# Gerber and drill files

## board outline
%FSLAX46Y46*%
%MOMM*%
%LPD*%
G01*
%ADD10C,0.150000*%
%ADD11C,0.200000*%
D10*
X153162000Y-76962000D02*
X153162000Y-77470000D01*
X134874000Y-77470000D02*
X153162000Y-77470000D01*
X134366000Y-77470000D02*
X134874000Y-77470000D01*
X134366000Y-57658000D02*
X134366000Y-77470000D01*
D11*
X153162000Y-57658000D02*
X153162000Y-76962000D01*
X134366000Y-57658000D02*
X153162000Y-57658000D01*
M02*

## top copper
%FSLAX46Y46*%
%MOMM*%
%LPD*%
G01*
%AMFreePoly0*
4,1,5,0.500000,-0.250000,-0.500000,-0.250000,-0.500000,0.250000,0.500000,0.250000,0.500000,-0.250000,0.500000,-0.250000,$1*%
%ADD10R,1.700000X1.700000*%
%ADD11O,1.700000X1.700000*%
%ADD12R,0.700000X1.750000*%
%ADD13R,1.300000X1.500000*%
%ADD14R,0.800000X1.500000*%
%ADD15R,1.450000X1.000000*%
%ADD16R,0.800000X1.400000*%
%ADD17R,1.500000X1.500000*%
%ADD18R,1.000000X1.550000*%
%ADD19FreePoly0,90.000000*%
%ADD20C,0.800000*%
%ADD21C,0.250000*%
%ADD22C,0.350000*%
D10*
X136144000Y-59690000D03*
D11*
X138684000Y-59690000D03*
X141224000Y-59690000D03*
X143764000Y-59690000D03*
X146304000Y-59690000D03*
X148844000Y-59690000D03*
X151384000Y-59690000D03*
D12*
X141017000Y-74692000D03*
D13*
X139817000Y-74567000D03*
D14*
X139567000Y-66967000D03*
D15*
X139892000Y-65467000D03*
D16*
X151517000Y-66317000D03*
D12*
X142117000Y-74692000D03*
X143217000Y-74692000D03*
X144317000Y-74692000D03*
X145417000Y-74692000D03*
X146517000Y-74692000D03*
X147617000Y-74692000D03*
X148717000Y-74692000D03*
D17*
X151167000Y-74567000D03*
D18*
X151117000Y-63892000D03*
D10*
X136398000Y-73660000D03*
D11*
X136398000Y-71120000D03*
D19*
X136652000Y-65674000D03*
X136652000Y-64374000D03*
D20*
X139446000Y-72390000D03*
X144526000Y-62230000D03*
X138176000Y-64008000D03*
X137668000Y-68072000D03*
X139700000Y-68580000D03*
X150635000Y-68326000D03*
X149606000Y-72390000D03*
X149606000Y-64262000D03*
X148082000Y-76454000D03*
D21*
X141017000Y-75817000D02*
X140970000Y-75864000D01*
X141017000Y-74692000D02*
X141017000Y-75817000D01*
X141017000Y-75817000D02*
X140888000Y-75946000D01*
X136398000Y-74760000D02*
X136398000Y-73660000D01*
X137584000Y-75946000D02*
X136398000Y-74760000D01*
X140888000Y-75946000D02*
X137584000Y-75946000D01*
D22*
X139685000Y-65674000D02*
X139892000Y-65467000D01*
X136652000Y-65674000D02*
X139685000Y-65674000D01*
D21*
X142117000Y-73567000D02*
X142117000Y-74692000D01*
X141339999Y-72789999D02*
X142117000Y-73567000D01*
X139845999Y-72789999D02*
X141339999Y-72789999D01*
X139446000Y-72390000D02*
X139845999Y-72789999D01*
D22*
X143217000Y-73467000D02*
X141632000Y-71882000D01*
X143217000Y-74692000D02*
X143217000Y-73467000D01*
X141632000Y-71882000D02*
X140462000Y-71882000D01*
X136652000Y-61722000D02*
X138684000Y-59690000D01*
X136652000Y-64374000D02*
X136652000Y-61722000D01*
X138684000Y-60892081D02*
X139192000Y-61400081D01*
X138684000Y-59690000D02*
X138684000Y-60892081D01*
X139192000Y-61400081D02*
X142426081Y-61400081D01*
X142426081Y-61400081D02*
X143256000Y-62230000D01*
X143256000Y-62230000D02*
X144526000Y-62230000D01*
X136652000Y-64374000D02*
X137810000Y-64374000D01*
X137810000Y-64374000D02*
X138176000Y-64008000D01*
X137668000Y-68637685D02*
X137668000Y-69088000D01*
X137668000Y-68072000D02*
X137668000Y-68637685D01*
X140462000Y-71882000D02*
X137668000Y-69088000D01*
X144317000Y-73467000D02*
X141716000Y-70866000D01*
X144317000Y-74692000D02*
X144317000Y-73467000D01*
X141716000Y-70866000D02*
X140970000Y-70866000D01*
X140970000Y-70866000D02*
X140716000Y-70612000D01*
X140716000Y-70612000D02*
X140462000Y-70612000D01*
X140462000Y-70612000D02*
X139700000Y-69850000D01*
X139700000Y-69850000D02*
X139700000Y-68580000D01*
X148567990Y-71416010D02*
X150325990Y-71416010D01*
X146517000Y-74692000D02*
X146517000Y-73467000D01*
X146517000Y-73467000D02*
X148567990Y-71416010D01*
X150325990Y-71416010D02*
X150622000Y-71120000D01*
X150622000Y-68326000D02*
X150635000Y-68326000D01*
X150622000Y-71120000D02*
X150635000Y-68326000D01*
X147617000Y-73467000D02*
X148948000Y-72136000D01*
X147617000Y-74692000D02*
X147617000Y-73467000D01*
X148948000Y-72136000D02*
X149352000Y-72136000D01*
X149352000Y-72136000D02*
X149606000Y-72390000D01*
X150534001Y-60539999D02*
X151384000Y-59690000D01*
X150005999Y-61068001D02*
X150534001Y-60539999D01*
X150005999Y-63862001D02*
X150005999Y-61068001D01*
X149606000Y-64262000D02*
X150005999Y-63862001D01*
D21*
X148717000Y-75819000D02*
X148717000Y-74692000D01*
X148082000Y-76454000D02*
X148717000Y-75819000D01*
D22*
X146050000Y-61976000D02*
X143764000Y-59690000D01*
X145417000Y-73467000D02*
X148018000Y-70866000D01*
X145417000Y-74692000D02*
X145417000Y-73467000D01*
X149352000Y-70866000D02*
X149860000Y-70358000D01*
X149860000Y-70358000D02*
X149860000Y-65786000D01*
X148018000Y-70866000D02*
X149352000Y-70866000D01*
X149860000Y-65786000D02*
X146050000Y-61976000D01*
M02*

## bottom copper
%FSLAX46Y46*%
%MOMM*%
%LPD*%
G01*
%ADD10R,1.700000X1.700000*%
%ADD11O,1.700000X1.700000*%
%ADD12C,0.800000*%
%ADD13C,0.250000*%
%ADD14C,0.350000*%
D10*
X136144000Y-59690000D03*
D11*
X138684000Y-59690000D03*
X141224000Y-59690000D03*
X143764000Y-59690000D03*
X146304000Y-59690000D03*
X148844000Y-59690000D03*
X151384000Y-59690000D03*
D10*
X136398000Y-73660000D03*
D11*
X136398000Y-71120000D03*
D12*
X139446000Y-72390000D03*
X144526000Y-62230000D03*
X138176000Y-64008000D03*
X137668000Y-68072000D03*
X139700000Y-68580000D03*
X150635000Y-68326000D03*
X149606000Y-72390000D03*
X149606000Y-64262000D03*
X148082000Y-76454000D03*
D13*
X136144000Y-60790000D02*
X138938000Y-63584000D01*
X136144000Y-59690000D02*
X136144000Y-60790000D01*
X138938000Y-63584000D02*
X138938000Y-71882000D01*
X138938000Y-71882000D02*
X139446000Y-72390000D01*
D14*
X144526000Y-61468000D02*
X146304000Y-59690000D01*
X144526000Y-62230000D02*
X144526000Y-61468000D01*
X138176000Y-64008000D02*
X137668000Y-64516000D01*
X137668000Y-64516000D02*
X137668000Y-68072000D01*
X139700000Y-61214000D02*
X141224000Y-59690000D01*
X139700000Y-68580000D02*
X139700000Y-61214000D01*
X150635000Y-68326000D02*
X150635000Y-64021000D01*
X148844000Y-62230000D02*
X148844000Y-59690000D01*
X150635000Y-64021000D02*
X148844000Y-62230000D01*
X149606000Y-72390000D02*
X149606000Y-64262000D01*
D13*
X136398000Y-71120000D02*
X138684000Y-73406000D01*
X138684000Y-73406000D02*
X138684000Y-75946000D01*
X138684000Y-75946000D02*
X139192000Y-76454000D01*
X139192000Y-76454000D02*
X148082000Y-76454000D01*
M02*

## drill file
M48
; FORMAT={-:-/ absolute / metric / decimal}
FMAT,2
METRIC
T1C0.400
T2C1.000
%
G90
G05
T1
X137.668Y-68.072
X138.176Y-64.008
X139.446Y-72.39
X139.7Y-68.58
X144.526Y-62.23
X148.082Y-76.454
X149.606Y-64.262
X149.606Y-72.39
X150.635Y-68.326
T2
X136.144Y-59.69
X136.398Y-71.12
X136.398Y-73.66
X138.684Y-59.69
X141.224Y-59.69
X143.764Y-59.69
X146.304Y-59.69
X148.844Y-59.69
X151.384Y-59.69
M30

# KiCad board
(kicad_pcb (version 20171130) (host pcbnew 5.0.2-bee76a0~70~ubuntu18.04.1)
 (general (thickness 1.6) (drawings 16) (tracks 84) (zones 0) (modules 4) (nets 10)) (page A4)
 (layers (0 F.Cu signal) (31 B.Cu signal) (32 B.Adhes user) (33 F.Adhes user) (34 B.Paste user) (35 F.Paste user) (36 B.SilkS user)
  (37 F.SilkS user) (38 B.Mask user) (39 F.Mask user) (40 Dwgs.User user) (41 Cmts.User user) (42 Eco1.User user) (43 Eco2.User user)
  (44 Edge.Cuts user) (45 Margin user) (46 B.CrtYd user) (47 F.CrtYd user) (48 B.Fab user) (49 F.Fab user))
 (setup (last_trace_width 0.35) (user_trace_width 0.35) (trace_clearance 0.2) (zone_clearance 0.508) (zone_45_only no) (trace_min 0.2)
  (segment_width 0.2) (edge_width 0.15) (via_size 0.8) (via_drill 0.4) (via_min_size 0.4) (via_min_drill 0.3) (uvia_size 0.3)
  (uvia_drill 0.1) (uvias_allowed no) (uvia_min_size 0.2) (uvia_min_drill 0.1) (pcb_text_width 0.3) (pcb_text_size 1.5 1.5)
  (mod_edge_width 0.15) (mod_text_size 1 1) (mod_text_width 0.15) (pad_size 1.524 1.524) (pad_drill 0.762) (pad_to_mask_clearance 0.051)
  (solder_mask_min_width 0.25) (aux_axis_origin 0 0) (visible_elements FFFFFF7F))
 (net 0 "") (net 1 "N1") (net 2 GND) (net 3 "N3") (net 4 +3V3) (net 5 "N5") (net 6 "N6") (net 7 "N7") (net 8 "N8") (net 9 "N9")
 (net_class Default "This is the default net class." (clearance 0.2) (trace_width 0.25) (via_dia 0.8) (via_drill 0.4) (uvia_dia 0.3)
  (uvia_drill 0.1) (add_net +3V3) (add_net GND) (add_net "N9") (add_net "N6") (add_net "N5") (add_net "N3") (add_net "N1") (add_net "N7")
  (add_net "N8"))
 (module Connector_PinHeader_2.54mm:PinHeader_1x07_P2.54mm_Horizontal (layer F.Cu) (at 136.144 59.69 90)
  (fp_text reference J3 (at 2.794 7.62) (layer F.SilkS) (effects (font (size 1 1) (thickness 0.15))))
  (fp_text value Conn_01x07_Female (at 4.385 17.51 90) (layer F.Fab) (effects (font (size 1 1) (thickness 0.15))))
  (pad 1 thru_hole rect (at 0 0 90) (size 1.7 1.7) (drill 1) (layers *.Cu *.Mask) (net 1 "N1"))
  (pad 2 thru_hole oval (at 0 2.54 90) (size 1.7 1.7) (drill 1) (layers *.Cu *.Mask) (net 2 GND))
  (pad 3 thru_hole oval (at 0 5.08 90) (size 1.7 1.7) (drill 1) (layers *.Cu *.Mask) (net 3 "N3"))
  (pad 4 thru_hole oval (at 0 7.62 90) (size 1.7 1.7) (drill 1) (layers *.Cu *.Mask) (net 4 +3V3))
  (pad 5 thru_hole oval (at 0 10.16 90) (size 1.7 1.7) (drill 1) (layers *.Cu *.Mask) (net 2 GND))
  (pad 6 thru_hole oval (at 0 12.7 90) (size 1.7 1.7) (drill 1) (layers *.Cu *.Mask) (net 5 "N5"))
  (pad 7 thru_hole oval (at 0 15.24 90) (size 1.7 1.7) (drill 1) (layers *.Cu *.Mask) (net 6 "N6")))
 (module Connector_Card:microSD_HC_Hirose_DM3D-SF (layer F.Cu) (at 145.542 69.342)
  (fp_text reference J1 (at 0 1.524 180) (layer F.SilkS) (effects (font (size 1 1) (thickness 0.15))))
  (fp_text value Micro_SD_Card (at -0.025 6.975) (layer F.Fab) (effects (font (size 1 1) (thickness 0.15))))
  (pad 8 smd rect (at -4.525 5.35) (size 0.7 1.75) (layers F.Cu F.Paste F.Mask) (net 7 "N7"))
  (pad 11 smd rect (at -5.725 5.225) (size 1.3 1.5) (layers F.Cu F.Paste F.Mask))
  (pad 11 smd rect (at -5.975 -2.375) (size 0.8 1.5) (layers F.Cu F.Paste F.Mask))
  (pad 9 smd rect (at -5.65 -3.875) (size 1.45 1) (layers F.Cu F.Paste F.Mask) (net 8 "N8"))
  (pad 11 smd rect (at 5.975 -3.025) (size 0.8 1.4) (layers F.Cu F.Paste F.Mask))
  (pad 7 smd rect (at -3.425 5.35) (size 0.7 1.75) (layers F.Cu F.Paste F.Mask) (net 1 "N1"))
  (pad 6 smd rect (at -2.325 5.35) (size 0.7 1.75) (layers F.Cu F.Paste F.Mask) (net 2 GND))
  (pad 5 smd rect (at -1.225 5.35) (size 0.7 1.75) (layers F.Cu F.Paste F.Mask) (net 3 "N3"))
  (pad 4 smd rect (at -0.125 5.35) (size 0.7 1.75) (layers F.Cu F.Paste F.Mask) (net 4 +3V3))
  (pad 3 smd rect (at 0.975 5.35) (size 0.7 1.75) (layers F.Cu F.Paste F.Mask) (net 5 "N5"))
  (pad 2 smd rect (at 2.075 5.35) (size 0.7 1.75) (layers F.Cu F.Paste F.Mask) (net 6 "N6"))
  (pad 1 smd rect (at 3.175 5.35) (size 0.7 1.75) (layers F.Cu F.Paste F.Mask) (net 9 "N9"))
  (pad 11 smd rect (at 5.625 5.225) (size 1.5 1.5) (layers F.Cu F.Paste F.Mask))
  (pad 10 smd rect (at 5.575 -5.45) (size 1 1.55) (layers F.Cu F.Paste F.Mask)))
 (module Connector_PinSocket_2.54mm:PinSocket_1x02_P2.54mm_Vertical (layer F.Cu) (at 136.398 73.66 180)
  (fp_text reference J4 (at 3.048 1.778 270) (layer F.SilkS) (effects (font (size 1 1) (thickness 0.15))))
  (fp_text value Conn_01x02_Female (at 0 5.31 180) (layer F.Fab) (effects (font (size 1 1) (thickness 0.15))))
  (pad 1 thru_hole rect (at 0 0 180) (size 1.7 1.7) (drill 1) (layers *.Cu *.Mask) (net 7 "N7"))
  (pad 2 thru_hole oval (at 0 2.54 180) (size 1.7 1.7) (drill 1) (layers *.Cu *.Mask) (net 9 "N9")))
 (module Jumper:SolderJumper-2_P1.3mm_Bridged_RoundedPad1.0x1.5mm (layer F.Cu) (at 136.652 65.024 90)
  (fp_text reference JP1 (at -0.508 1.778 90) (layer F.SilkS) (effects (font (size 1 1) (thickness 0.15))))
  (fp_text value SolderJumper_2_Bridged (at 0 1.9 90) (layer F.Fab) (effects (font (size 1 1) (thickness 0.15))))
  (pad 1 smd custom (at -0.65 0 90) (size 1 0.5) (layers F.Cu F.Mask) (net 8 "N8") (zone_connect 0)
   (options (clearance outline) (anchor rect)) (primitives))
  (pad 2 smd custom (at 0.65 0 90) (size 1 0.5) (layers F.Cu F.Mask) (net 2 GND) (zone_connect 0)
   (options (clearance outline) (anchor rect)) (primitives)))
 (gr_line (start 153.162 76.962) (end 153.162 77.47) (layer Edge.Cuts) (width 0.15))
 (gr_line (start 134.874 77.47) (end 153.162 77.47) (layer Edge.Cuts) (width 0.15))
 (gr_line (start 134.366 77.47) (end 134.874 77.47) (layer Edge.Cuts) (width 0.15))
 (gr_line (start 134.366 57.658) (end 134.366 77.47) (layer Edge.Cuts) (width 0.15))
 (gr_line (start 153.162 57.658) (end 153.162 76.962) (layer Edge.Cuts) (width 0.2))
 (gr_line (start 134.366 57.658) (end 153.162 57.658) (layer Edge.Cuts) (width 0.2))
 (segment (start 141.017 75.817) (end 140.97 75.864) (width 0.25) (layer F.Cu) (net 7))
 (segment (start 141.017 74.692) (end 141.017 75.817) (width 0.25) (layer F.Cu) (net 7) (status 10))
 (segment (start 141.017 75.817) (end 140.888 75.946) (width 0.25) (layer F.Cu) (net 7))
 (segment (start 136.398 74.76) (end 136.398 73.66) (width 0.25) (layer F.Cu) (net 7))
 (segment (start 137.584 75.946) (end 136.398 74.76) (width 0.25) (layer F.Cu) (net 7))
 (segment (start 140.888 75.946) (end 137.584 75.946) (width 0.25) (layer F.Cu) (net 7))
 (segment (start 139.685 65.674) (end 139.892 65.467) (width 0.35) (layer F.Cu) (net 8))
 (segment (start 136.652 65.674) (end 139.685 65.674) (width 0.35) (layer F.Cu) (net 8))
 (segment (start 136.144 60.79) (end 138.938 63.584) (width 0.25) (layer B.Cu) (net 1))
 (segment (start 136.144 59.69) (end 136.144 60.79) (width 0.25) (layer B.Cu) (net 1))
 (via (at 139.446 72.39) (size 0.8) (drill 0.4) (layers F.Cu B.Cu) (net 1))
 (segment (start 138.938 63.584) (end 138.938 71.882) (width 0.25) (layer B.Cu) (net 1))
 (segment (start 138.938 71.882) (end 139.446 72.39) (width 0.25) (layer B.Cu) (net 1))
 (segment (start 142.117 73.567) (end 142.117 74.692) (width 0.25) (layer F.Cu) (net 1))
 (segment (start 141.339999 72.789999) (end 142.117 73.567) (width 0.25) (layer F.Cu) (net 1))
 (segment (start 139.845999 72.789999) (end 141.339999 72.789999) (width 0.25) (layer F.Cu) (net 1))
 (segment (start 139.446 72.39) (end 139.845999 72.789999) (width 0.25) (layer F.Cu) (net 1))
 (segment (start 143.217 73.467) (end 141.632 71.882) (width 0.35) (layer F.Cu) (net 2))
 (segment (start 143.217 74.692) (end 143.217 73.467) (width 0.35) (layer F.Cu) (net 2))
 (segment (start 141.632 71.882) (end 140.462 71.882) (width 0.35) (layer F.Cu) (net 2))
 (segment (start 136.652 61.722) (end 138.684 59.69) (width 0.35) (layer F.Cu) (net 2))
 (segment (start 136.652 64.374) (end 136.652 61.722) (width 0.35) (layer F.Cu) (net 2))
 (segment (start 138.684 60.892081) (end 139.192 61.400081) (width 0.35) (layer F.Cu) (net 2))
 (segment (start 138.684 59.69) (end 138.684 60.892081) (width 0.35) (layer F.Cu) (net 2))
 (segment (start 139.192 61.400081) (end 142.426081 61.400081) (width 0.35) (layer F.Cu) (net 2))
 (segment (start 142.426081 61.400081) (end 143.256 62.23) (width 0.35) (layer F.Cu) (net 2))
 (via (at 144.526 62.23) (size 0.8) (drill 0.4) (layers F.Cu B.Cu) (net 2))
 (segment (start 143.256 62.23) (end 144.526 62.23) (width 0.35) (layer F.Cu) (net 2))
 (segment (start 144.526 61.468) (end 146.304 59.69) (width 0.35) (layer B.Cu) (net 2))
 (segment (start 144.526 62.23) (end 144.526 61.468) (width 0.35) (layer B.Cu) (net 2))
 (via (at 138.176 64.008) (size 0.8) (drill 0.4) (layers F.Cu B.Cu) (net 2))
 (segment (start 136.652 64.374) (end 137.81 64.374) (width 0.35) (layer F.Cu) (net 2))
 (segment (start 137.81 64.374) (end 138.176 64.008) (width 0.35) (layer F.Cu) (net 2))
 (via (at 137.668 68.072) (size 0.8) (drill 0.4) (layers F.Cu B.Cu) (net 2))
 (segment (start 138.176 64.008) (end 137.668 64.516) (width 0.35) (layer B.Cu) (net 2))
 (segment (start 137.668 64.516) (end 137.668 68.072) (width 0.35) (layer B.Cu) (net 2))
 (segment (start 137.668 68.637685) (end 137.668 69.088) (width 0.35) (layer F.Cu) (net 2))
 (segment (start 137.668 68.072) (end 137.668 68.637685) (width 0.35) (layer F.Cu) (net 2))
 (segment (start 140.462 71.882) (end 137.668 69.088) (width 0.35) (layer F.Cu) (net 2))
 (segment (start 144.317 73.467) (end 141.716 70.866) (width 0.35) (layer F.Cu) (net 3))
 (segment (start 144.317 74.692) (end 144.317 73.467) (width 0.35) (layer F.Cu) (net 3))
 (segment (start 141.716 70.866) (end 140.97 70.866) (width 0.35) (layer F.Cu) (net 3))
 (segment (start 140.97 70.866) (end 140.716 70.612) (width 0.35) (layer F.Cu) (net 3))
 (segment (start 140.716 70.612) (end 140.462 70.612) (width 0.35) (layer F.Cu) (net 3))
 (via (at 139.7 68.58) (size 0.8) (drill 0.4) (layers F.Cu B.Cu) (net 3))
 (segment (start 140.462 70.612) (end 139.7 69.85) (width 0.35) (layer F.Cu) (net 3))
 (segment (start 139.7 69.85) (end 139.7 68.58) (width 0.35) (layer F.Cu) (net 3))
 (segment (start 139.7 61.214) (end 141.224 59.69) (width 0.35) (layer B.Cu) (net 3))
 (segment (start 139.7 68.58) (end 139.7 61.214) (width 0.35) (layer B.Cu) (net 3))
 (segment (start 148.56799 71.41601) (end 150.32599 71.41601) (width 0.35) (layer F.Cu) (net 5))
 (segment (start 146.517 74.692) (end 146.517 73.467) (width 0.35) (layer F.Cu) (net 5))
 (segment (start 146.517 73.467) (end 148.56799 71.41601) (width 0.35) (layer F.Cu) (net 5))
 (segment (start 150.32599 71.41601) (end 150.622 71.12) (width 0.35) (layer F.Cu) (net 5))
 (via (at 150.635 68.326) (size 0.8) (drill 0.4) (layers F.Cu B.Cu) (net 5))
 (segment (start 150.622 68.326) (end 150.635 68.326) (width 0.35) (layer F.Cu) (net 5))
 (segment (start 150.622 71.12) (end 150.635 68.326) (width 0.35) (layer F.Cu) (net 5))
 (segment (start 150.635 68.326) (end 150.635 64.021) (width 0.35) (layer B.Cu) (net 5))
 (segment (start 148.844 62.23) (end 148.844 59.69) (width 0.35) (layer B.Cu) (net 5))
 (segment (start 150.635 64.021) (end 148.844 62.23) (width 0.35) (layer B.Cu) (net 5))
 (segment (start 147.617 73.467) (end 148.948 72.136) (width 0.35) (layer F.Cu) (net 6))
 (segment (start 147.617 74.692) (end 147.617 73.467) (width 0.35) (layer F.Cu) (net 6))
 (via (at 149.606 72.39) (size 0.8) (drill 0.4) (layers F.Cu B.Cu) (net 6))
 (segment (start 148.948 72.136) (end 149.352 72.136) (width 0.35) (layer F.Cu) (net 6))
 (segment (start 149.352 72.136) (end 149.606 72.39) (width 0.35) (layer F.Cu) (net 6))
 (via (at 149.606 64.262) (size 0.8) (drill 0.4) (layers F.Cu B.Cu) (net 6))
 (segment (start 149.606 72.39) (end 149.606 64.262) (width 0.35) (layer B.Cu) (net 6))
 (segment (start 150.534001 60.539999) (end 151.384 59.69) (width 0.35) (layer F.Cu) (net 6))
 (segment (start 150.005999 61.068001) (end 150.534001 60.539999) (width 0.35) (layer F.Cu) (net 6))
 (segment (start 150.005999 63.862001) (end 150.005999 61.068001) (width 0.35) (layer F.Cu) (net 6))
 (segment (start 149.606 64.262) (end 150.005999 63.862001) (width 0.35) (layer F.Cu) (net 6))
 (segment (start 136.398 71.12) (end 138.684 73.406) (width 0.25) (layer B.Cu) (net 9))
 (segment (start 138.684 73.406) (end 138.684 75.946) (width 0.25) (layer B.Cu) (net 9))
 (via (at 148.082 76.454) (size 0.8) (drill 0.4) (layers F.Cu B.Cu) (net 9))
 (segment (start 138.684 75.946) (end 139.192 76.454) (width 0.25) (layer B.Cu) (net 9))
 (segment (start 139.192 76.454) (end 148.082 76.454) (width 0.25) (layer B.Cu) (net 9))
 (segment (start 148.717 75.819) (end 148.717 74.692) (width 0.25) (layer F.Cu) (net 9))
 (segment (start 148.082 76.454) (end 148.717 75.819) (width 0.25) (layer F.Cu) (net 9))
 (segment (start 146.05 61.976) (end 143.764 59.69) (width 0.35) (layer F.Cu) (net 4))
 (segment (start 145.417 73.467) (end 148.018 70.866) (width 0.35) (layer F.Cu) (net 4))
 (segment (start 145.417 74.692) (end 145.417 73.467) (width 0.35) (layer F.Cu) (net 4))
 (segment (start 149.352 70.866) (end 149.86 70.358) (width 0.35) (layer F.Cu) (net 4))
 (segment (start 149.86 70.358) (end 149.86 65.786) (width 0.35) (layer F.Cu) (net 4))
 (segment (start 148.018 70.866) (end 149.352 70.866) (width 0.35) (layer F.Cu) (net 4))
 (segment (start 149.86 65.786) (end 146.05 61.976) (width 0.35) (layer F.Cu) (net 4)))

